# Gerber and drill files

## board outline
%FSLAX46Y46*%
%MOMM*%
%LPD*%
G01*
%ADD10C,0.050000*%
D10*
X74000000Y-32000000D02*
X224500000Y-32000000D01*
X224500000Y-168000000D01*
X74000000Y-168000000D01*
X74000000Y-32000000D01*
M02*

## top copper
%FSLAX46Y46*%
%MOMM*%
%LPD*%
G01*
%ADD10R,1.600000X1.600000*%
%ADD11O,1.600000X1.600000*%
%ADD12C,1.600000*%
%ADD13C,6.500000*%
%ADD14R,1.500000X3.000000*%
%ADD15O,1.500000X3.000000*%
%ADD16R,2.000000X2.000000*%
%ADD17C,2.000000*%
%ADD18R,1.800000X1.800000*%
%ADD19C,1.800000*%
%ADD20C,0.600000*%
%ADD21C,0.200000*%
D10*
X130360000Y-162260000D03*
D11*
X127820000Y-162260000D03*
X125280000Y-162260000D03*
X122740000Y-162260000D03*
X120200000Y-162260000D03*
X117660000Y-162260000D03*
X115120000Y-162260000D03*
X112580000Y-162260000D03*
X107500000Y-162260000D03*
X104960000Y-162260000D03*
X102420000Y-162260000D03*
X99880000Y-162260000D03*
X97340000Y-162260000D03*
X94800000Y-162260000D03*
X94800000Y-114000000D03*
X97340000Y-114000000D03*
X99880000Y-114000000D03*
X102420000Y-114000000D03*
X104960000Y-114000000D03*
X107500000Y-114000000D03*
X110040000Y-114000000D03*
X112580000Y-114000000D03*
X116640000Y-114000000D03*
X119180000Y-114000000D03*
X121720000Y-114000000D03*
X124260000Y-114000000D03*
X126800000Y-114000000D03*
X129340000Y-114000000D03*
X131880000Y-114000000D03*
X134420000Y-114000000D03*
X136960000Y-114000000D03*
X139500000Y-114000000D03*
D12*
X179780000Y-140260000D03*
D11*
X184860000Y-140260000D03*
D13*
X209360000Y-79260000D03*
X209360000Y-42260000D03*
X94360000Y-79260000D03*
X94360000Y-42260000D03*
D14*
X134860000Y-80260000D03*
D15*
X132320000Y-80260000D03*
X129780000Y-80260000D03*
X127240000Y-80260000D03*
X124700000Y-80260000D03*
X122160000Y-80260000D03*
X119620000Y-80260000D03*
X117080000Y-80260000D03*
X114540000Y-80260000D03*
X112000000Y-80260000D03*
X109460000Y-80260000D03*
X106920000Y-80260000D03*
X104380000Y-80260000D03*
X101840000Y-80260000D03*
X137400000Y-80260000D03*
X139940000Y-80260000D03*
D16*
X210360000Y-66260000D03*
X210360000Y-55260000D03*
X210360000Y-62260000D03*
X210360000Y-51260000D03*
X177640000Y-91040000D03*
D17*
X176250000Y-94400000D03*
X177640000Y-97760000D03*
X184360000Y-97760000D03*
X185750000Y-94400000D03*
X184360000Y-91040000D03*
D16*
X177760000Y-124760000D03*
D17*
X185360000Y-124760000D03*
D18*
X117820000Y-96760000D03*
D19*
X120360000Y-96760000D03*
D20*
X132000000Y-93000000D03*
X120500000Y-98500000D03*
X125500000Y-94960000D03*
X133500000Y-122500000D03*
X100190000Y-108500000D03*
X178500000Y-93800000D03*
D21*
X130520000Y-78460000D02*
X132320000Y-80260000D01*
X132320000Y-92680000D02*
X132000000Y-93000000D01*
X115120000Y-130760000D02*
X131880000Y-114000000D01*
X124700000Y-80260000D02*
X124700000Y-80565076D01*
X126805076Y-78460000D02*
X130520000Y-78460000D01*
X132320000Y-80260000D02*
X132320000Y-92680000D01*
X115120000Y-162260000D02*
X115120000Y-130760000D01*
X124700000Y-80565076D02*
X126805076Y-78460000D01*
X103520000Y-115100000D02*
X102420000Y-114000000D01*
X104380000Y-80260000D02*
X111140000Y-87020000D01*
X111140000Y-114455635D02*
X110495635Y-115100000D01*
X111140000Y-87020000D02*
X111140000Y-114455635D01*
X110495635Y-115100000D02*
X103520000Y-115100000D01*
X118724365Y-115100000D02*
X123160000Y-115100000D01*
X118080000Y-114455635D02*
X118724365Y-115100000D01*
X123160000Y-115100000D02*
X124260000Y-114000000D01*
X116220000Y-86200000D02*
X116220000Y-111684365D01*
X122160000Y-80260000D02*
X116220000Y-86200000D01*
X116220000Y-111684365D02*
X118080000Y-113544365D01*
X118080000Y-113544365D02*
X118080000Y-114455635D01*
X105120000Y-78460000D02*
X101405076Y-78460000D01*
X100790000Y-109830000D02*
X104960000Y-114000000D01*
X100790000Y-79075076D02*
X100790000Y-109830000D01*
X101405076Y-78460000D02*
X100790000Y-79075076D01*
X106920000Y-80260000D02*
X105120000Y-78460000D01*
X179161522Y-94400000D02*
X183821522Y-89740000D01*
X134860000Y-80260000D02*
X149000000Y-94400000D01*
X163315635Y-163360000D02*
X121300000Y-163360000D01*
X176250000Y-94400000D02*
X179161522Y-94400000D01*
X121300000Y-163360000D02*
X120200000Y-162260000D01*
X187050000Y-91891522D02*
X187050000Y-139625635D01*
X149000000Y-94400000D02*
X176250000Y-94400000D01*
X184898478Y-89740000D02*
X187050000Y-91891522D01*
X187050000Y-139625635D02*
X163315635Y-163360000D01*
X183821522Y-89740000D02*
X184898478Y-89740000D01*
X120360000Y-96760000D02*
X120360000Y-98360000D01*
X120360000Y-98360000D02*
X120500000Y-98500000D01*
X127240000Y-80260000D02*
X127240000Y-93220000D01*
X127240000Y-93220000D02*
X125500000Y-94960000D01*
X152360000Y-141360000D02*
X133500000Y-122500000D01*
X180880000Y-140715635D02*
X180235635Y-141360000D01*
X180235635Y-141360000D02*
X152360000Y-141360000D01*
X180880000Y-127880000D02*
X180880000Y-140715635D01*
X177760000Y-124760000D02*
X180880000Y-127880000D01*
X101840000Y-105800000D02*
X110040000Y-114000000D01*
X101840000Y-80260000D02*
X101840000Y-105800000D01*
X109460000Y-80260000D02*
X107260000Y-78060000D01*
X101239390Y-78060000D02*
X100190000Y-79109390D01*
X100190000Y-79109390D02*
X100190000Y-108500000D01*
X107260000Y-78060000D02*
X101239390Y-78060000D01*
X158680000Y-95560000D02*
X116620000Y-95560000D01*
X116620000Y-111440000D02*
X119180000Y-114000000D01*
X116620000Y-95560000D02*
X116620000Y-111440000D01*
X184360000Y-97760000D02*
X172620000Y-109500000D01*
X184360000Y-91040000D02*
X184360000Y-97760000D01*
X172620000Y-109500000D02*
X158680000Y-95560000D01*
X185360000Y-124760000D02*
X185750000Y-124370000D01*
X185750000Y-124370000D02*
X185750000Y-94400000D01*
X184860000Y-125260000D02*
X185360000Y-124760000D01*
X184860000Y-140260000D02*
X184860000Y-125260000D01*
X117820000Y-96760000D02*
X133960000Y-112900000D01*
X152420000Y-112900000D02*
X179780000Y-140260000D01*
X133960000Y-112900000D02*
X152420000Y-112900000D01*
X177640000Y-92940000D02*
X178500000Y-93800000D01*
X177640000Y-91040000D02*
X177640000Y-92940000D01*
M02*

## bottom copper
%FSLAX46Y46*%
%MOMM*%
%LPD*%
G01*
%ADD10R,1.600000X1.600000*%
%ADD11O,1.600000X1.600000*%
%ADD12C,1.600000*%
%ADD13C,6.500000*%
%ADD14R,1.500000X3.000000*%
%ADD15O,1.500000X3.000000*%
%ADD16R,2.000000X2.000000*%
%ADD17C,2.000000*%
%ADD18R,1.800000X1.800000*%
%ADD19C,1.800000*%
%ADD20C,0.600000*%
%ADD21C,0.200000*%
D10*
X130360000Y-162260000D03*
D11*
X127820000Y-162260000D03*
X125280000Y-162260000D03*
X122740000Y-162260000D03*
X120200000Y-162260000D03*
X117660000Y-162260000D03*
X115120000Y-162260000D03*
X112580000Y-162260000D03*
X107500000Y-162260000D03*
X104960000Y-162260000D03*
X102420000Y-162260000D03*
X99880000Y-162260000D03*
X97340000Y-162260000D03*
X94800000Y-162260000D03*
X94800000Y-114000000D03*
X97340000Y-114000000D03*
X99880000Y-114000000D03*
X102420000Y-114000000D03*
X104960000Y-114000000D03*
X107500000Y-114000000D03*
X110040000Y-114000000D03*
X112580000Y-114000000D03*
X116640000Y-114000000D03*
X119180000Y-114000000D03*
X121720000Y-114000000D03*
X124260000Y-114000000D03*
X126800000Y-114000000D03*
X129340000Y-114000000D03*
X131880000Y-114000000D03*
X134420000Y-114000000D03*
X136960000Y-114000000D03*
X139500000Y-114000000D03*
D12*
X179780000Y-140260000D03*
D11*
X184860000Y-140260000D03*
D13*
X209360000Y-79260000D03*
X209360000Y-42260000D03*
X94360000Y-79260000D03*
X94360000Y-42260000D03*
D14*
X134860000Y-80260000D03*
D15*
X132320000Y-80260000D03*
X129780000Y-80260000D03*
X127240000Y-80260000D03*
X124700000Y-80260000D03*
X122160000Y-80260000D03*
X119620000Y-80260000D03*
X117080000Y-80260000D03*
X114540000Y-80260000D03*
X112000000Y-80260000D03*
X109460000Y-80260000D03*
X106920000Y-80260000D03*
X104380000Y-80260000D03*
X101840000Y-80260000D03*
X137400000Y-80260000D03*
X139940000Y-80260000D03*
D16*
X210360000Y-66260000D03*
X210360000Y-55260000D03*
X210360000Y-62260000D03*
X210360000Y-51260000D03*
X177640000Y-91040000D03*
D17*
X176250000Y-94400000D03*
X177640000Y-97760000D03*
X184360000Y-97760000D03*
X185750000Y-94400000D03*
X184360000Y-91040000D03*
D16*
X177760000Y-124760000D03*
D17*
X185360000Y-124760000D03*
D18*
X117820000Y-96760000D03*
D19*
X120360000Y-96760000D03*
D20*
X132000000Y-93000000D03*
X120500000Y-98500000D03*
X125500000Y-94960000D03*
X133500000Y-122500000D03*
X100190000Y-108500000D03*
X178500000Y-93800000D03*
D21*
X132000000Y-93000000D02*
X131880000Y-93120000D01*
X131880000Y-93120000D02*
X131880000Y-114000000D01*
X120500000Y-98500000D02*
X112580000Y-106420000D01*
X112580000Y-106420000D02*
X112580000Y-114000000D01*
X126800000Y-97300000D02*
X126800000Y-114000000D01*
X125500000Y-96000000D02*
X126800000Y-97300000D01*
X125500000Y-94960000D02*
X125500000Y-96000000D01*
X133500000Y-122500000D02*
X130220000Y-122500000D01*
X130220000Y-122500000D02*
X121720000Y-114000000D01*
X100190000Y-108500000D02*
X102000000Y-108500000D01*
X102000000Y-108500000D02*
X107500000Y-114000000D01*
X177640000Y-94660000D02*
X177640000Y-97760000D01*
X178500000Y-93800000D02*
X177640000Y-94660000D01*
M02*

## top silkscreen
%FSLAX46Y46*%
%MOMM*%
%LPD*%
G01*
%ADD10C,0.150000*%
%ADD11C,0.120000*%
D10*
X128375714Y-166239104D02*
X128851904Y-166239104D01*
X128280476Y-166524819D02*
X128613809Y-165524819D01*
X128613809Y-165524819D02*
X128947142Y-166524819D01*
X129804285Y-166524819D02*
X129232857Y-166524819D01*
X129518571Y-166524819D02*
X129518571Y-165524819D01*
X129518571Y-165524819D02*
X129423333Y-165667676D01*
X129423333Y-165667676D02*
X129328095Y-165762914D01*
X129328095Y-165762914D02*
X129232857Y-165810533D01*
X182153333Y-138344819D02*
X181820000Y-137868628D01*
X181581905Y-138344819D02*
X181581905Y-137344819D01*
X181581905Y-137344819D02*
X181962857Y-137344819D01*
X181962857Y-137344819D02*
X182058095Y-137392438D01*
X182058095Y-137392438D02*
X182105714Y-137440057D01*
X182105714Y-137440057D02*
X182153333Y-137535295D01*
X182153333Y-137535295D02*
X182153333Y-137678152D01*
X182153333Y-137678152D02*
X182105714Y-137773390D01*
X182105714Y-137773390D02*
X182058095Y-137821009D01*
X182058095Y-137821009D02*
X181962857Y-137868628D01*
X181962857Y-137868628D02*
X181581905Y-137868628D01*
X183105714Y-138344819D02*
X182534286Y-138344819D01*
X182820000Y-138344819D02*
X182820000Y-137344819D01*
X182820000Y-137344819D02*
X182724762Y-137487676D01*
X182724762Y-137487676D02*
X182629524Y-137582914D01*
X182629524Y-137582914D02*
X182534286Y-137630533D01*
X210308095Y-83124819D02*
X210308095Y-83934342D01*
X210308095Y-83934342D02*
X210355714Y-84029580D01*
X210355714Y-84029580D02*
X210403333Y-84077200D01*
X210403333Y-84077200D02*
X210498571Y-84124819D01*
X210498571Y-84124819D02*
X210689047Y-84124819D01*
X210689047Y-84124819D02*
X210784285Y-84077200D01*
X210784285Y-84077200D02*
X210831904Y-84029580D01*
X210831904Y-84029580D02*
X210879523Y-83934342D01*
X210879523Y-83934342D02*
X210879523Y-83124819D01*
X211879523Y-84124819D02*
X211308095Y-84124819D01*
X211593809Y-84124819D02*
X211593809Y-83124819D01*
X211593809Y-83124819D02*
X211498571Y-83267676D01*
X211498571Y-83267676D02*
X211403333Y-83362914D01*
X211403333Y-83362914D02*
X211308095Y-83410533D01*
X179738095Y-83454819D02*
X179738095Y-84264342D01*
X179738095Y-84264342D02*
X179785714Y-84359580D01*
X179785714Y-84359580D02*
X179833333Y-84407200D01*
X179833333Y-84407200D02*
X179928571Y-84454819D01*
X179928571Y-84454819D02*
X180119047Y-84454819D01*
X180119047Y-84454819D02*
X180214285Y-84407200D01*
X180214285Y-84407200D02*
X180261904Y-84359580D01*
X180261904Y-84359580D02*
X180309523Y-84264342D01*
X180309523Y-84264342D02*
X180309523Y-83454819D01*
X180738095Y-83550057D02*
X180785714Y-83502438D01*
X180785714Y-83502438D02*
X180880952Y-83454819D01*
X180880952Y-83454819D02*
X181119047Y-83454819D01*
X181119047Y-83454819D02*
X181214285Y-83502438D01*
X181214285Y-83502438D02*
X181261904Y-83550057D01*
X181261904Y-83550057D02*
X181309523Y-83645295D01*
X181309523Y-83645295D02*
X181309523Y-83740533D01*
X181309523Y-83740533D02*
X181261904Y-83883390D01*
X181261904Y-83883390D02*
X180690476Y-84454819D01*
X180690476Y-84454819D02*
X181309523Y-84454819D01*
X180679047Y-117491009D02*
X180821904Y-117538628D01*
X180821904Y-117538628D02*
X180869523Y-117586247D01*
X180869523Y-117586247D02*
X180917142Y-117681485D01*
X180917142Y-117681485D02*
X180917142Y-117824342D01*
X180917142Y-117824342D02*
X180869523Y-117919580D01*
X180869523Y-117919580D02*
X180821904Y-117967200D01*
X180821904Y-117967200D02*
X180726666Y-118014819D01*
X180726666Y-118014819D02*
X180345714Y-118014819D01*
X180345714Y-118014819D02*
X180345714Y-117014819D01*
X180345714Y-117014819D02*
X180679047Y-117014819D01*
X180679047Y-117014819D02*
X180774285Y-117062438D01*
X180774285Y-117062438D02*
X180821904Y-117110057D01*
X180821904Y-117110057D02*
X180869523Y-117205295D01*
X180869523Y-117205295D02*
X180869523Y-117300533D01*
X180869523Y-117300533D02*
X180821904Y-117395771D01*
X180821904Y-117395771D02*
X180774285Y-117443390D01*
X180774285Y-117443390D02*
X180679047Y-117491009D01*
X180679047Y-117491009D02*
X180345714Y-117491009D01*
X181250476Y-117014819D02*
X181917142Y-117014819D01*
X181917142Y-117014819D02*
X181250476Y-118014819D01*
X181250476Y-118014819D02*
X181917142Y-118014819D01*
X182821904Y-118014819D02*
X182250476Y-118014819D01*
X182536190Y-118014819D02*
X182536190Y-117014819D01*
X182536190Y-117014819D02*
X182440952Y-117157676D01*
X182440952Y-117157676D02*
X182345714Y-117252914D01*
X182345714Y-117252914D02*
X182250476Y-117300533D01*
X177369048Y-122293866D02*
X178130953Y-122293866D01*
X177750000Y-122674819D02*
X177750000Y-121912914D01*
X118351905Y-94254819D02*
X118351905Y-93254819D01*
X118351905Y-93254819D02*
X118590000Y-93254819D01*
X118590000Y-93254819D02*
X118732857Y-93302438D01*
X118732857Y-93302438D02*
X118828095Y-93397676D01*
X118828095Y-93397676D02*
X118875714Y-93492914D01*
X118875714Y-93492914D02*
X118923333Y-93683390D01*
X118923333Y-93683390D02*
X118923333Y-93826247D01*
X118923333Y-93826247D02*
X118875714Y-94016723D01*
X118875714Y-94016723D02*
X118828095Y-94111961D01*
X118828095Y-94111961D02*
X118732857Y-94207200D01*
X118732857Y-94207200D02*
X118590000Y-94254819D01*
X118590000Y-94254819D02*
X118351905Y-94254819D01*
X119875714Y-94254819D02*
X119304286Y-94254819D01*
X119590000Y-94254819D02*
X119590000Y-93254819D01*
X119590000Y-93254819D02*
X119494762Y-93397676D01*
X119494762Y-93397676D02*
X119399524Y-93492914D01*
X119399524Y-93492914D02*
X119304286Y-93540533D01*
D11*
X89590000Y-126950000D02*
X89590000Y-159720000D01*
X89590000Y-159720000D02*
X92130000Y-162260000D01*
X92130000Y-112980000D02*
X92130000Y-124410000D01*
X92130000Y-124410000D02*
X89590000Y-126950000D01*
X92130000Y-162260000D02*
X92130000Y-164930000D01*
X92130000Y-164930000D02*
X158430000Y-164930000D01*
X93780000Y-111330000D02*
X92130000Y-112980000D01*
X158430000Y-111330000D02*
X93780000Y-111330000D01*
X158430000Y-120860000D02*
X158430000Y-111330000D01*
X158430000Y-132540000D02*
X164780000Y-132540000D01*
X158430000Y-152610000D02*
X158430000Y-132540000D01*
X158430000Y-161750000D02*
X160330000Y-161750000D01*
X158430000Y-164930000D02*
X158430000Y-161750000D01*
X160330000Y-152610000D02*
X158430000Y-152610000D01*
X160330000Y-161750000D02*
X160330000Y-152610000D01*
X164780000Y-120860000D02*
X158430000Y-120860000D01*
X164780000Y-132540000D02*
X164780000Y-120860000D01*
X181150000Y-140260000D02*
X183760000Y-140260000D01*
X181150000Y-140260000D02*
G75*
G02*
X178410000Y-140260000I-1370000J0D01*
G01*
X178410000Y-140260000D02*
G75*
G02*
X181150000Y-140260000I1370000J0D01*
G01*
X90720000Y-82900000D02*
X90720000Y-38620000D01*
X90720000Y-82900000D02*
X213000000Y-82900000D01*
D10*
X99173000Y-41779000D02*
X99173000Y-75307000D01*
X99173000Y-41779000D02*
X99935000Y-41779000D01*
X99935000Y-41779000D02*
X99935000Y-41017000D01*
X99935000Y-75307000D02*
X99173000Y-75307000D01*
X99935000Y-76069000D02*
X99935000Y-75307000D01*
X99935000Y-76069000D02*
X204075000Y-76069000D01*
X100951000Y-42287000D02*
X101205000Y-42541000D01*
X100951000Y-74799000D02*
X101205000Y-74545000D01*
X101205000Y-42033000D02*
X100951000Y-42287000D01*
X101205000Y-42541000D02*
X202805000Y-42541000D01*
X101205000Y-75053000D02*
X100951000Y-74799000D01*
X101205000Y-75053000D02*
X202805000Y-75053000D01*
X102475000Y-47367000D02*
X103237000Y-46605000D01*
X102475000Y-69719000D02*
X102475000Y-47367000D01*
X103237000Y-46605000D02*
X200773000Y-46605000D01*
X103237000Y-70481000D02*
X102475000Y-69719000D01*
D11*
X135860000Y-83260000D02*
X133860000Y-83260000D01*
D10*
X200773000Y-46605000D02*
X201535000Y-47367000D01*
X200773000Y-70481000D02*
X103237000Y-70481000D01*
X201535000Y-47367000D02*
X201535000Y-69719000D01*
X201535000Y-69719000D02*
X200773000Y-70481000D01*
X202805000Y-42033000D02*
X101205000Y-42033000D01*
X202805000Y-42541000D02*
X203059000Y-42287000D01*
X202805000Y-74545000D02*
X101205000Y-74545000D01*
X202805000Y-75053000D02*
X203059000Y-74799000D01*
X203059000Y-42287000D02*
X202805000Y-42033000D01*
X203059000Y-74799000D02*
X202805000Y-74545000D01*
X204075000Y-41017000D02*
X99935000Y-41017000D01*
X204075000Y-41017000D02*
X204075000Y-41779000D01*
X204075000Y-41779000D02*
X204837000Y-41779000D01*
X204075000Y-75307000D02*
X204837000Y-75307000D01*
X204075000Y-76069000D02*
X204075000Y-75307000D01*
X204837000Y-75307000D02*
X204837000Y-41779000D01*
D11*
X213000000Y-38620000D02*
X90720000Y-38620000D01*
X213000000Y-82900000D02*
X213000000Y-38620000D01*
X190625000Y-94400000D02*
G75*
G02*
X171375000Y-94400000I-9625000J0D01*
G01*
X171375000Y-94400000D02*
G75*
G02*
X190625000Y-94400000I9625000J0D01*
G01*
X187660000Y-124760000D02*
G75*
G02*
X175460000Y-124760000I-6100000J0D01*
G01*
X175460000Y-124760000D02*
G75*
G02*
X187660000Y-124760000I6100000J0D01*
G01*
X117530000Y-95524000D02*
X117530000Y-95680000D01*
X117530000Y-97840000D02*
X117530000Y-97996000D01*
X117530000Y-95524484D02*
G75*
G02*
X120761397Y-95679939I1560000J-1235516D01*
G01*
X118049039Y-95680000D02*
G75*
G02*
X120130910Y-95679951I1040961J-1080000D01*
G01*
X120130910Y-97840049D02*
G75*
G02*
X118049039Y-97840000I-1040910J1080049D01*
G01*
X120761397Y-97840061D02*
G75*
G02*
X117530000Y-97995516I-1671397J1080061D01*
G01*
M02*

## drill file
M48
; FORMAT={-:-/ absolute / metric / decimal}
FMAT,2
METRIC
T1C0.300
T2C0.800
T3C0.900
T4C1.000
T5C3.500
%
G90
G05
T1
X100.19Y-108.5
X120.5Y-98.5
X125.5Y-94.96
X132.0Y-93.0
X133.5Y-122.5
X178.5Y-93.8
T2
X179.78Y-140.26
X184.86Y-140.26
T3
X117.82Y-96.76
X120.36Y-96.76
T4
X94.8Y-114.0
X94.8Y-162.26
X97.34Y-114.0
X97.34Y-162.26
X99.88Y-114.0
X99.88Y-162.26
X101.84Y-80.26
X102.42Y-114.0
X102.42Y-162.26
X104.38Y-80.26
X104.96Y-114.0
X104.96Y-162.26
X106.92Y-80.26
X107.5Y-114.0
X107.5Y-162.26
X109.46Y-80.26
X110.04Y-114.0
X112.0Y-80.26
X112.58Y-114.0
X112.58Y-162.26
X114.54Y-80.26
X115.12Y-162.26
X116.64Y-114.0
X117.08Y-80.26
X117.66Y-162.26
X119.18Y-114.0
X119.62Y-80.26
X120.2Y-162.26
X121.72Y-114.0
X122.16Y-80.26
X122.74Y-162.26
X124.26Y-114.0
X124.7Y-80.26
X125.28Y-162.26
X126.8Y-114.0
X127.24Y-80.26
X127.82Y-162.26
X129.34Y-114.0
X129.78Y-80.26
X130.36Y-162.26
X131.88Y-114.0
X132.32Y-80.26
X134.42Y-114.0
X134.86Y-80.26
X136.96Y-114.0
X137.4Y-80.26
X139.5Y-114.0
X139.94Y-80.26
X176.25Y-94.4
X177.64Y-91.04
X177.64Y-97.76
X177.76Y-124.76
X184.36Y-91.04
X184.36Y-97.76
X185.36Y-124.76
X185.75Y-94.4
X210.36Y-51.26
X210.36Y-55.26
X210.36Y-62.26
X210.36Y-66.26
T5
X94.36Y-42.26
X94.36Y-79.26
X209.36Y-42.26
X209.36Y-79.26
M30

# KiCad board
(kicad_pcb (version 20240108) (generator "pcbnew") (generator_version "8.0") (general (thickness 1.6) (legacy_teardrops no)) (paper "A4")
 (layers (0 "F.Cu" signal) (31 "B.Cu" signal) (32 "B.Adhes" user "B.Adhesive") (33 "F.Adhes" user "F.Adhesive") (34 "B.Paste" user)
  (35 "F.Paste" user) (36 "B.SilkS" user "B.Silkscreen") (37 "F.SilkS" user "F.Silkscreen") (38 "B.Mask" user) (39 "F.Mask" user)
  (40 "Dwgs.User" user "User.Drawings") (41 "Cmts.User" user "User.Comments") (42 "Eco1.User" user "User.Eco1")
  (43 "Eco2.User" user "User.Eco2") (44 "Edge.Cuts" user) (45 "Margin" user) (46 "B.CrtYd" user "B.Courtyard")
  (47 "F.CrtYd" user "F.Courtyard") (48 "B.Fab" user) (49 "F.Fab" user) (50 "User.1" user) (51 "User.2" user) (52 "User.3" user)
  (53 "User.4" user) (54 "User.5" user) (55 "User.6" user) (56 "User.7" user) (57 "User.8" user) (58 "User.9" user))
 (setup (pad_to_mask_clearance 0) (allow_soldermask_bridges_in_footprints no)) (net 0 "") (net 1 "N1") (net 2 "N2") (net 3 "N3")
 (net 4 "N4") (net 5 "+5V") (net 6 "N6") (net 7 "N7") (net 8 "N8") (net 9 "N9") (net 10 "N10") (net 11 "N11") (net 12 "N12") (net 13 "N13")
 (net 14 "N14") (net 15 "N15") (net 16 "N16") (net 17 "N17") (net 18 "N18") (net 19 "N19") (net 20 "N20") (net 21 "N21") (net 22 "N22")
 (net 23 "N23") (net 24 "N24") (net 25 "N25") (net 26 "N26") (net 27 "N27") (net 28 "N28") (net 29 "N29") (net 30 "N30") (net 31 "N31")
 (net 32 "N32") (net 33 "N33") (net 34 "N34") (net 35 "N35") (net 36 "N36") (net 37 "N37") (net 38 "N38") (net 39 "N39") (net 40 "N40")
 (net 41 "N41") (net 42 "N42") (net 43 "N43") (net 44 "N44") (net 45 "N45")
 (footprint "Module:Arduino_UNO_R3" (layer "F.Cu") (at 130.36 162.26 180)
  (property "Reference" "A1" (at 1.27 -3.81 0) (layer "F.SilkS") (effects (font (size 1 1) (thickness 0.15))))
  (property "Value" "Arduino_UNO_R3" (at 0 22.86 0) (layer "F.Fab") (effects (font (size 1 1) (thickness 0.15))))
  (fp_line (start 40.77 35.31) (end 40.77 2.54) (stroke (width 0.12) (type solid)) (layer "F.SilkS"))
  (fp_line (start 40.77 2.54) (end 38.23 0) (stroke (width 0.12) (type solid)) (layer "F.SilkS"))
  (fp_line (start 38.23 49.28) (end 38.23 37.85) (stroke (width 0.12) (type solid)) (layer "F.SilkS"))
  (fp_line (start 38.23 37.85) (end 40.77 35.31) (stroke (width 0.12) (type solid)) (layer "F.SilkS"))
  (fp_line (start 38.23 0) (end 38.23 -2.67) (stroke (width 0.12) (type solid)) (layer "F.SilkS"))
  (fp_line (start 38.23 -2.67) (end -28.07 -2.67) (stroke (width 0.12) (type solid)) (layer "F.SilkS"))
  (fp_line (start 36.58 50.93) (end 38.23 49.28) (stroke (width 0.12) (type solid)) (layer "F.SilkS"))
  (fp_line (start -28.07 50.93) (end 36.58 50.93) (stroke (width 0.12) (type solid)) (layer "F.SilkS"))
  (fp_line (start -28.07 41.4) (end -28.07 50.93) (stroke (width 0.12) (type solid)) (layer "F.SilkS"))
  (fp_line (start -28.07 29.72) (end -34.42 29.72) (stroke (width 0.12) (type solid)) (layer "F.SilkS"))
  (fp_line (start -28.07 9.65) (end -28.07 29.72) (stroke (width 0.12) (type solid)) (layer "F.SilkS"))
  (fp_line (start -28.07 0.51) (end -29.97 0.51) (stroke (width 0.12) (type solid)) (layer "F.SilkS"))
  (fp_line (start -28.07 -2.67) (end -28.07 0.51) (stroke (width 0.12) (type solid)) (layer "F.SilkS"))
  (fp_line (start -29.97 9.65) (end -28.07 9.65) (stroke (width 0.12) (type solid)) (layer "F.SilkS"))
  (fp_line (start -29.97 0.51) (end -29.97 9.65) (stroke (width 0.12) (type solid)) (layer "F.SilkS"))
  (fp_line (start -34.42 41.4) (end -28.07 41.4) (stroke (width 0.12) (type solid)) (layer "F.SilkS"))
  (fp_line (start -34.42 29.72) (end -34.42 41.4) (stroke (width 0.12) (type solid)) (layer "F.SilkS"))
  (pad "1" thru_hole rect (at 0 0 270) (size 1.6 1.6) (drill 1) (layers "*.Cu" "*.Mask") (remove_unused_layers no) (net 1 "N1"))
  (pad "2" thru_hole oval (at 2.54 0 270) (size 1.6 1.6) (drill 1) (layers "*.Cu" "*.Mask") (remove_unused_layers no) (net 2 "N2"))
  (pad "3" thru_hole oval (at 5.08 0 270) (size 1.6 1.6) (drill 1) (layers "*.Cu" "*.Mask") (remove_unused_layers no) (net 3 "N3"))
  (pad "4" thru_hole oval (at 7.62 0 270) (size 1.6 1.6) (drill 1) (layers "*.Cu" "*.Mask") (remove_unused_layers no) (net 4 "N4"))
  (pad "5" thru_hole oval (at 10.16 0 270) (size 1.6 1.6) (drill 1) (layers "*.Cu" "*.Mask") (remove_unused_layers no) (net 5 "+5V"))
  (pad "6" thru_hole oval (at 12.7 0 270) (size 1.6 1.6) (drill 1) (layers "*.Cu" "*.Mask") (remove_unused_layers no) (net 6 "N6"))
  (pad "7" thru_hole oval (at 15.24 0 270) (size 1.6 1.6) (drill 1) (layers "*.Cu" "*.Mask") (remove_unused_layers no) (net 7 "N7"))
  (pad "8" thru_hole oval (at 17.78 0 270) (size 1.6 1.6) (drill 1) (layers "*.Cu" "*.Mask") (remove_unused_layers no) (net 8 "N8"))
  (pad "9" thru_hole oval (at 22.86 0 270) (size 1.6 1.6) (drill 1) (layers "*.Cu" "*.Mask") (remove_unused_layers no) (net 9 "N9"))
  (pad "10" thru_hole oval (at 25.4 0 270) (size 1.6 1.6) (drill 1) (layers "*.Cu" "*.Mask") (remove_unused_layers no) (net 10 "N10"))
  (pad "11" thru_hole oval (at 27.94 0 270) (size 1.6 1.6) (drill 1) (layers "*.Cu" "*.Mask") (remove_unused_layers no) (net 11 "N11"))
  (pad "12" thru_hole oval (at 30.48 0 270) (size 1.6 1.6) (drill 1) (layers "*.Cu" "*.Mask") (remove_unused_layers no) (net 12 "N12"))
  (pad "13" thru_hole oval (at 33.02 0 270) (size 1.6 1.6) (drill 1) (layers "*.Cu" "*.Mask") (remove_unused_layers no) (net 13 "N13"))
  (pad "14" thru_hole oval (at 35.56 0 270) (size 1.6 1.6) (drill 1) (layers "*.Cu" "*.Mask") (remove_unused_layers no) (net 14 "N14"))
  (pad "15" thru_hole oval (at 35.56 48.26 270) (size 1.6 1.6) (drill 1) (layers "*.Cu" "*.Mask") (remove_unused_layers no) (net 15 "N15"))
  (pad "16" thru_hole oval (at 33.02 48.26 270) (size 1.6 1.6) (drill 1) (layers "*.Cu" "*.Mask") (remove_unused_layers no) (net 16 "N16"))
  (pad "17" thru_hole oval (at 30.48 48.26 270) (size 1.6 1.6) (drill 1) (layers "*.Cu" "*.Mask") (remove_unused_layers no) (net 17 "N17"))
  (pad "18" thru_hole oval (at 27.94 48.26 270) (size 1.6 1.6) (drill 1) (layers "*.Cu" "*.Mask") (remove_unused_layers no) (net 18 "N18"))
  (pad "19" thru_hole oval (at 25.4 48.26 270) (size 1.6 1.6) (drill 1) (layers "*.Cu" "*.Mask") (remove_unused_layers no) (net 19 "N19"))
  (pad "20" thru_hole oval (at 22.86 48.26 270) (size 1.6 1.6) (drill 1) (layers "*.Cu" "*.Mask") (remove_unused_layers no) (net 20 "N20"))
  (pad "21" thru_hole oval (at 20.32 48.26 270) (size 1.6 1.6) (drill 1) (layers "*.Cu" "*.Mask") (remove_unused_layers no) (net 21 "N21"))
  (pad "22" thru_hole oval (at 17.78 48.26 270) (size 1.6 1.6) (drill 1) (layers "*.Cu" "*.Mask") (remove_unused_layers no) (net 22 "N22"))
  (pad "23" thru_hole oval (at 13.72 48.26 270) (size 1.6 1.6) (drill 1) (layers "*.Cu" "*.Mask") (remove_unused_layers no) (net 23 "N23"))
  (pad "24" thru_hole oval (at 11.18 48.26 270) (size 1.6 1.6) (drill 1) (layers "*.Cu" "*.Mask") (remove_unused_layers no) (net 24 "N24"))
  (pad "25" thru_hole oval (at 8.64 48.26 270) (size 1.6 1.6) (drill 1) (layers "*.Cu" "*.Mask") (remove_unused_layers no) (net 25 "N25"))
  (pad "26" thru_hole oval (at 6.1 48.26 270) (size 1.6 1.6) (drill 1) (layers "*.Cu" "*.Mask") (remove_unused_layers no) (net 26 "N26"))
  (pad "27" thru_hole oval (at 3.56 48.26 270) (size 1.6 1.6) (drill 1) (layers "*.Cu" "*.Mask") (remove_unused_layers no) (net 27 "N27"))
  (pad "28" thru_hole oval (at 1.02 48.26 270) (size 1.6 1.6) (drill 1) (layers "*.Cu" "*.Mask") (remove_unused_layers no) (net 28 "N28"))
  (pad "29" thru_hole oval (at -1.52 48.26 270) (size 1.6 1.6) (drill 1) (layers "*.Cu" "*.Mask") (remove_unused_layers no) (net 7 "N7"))
  (pad "30" thru_hole oval (at -4.06 48.26 270) (size 1.6 1.6) (drill 1) (layers "*.Cu" "*.Mask") (remove_unused_layers no) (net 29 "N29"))
  (pad "31" thru_hole oval (at -6.6 48.26 270) (size 1.6 1.6) (drill 1) (layers "*.Cu" "*.Mask") (remove_unused_layers no) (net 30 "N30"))
  (pad "32" thru_hole oval (at -9.14 48.26 270) (size 1.6 1.6) (drill 1) (layers "*.Cu" "*.Mask") (remove_unused_layers no) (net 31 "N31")))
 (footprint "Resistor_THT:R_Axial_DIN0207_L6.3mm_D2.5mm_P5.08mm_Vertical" (layer "F.Cu") (at 179.78 140.26)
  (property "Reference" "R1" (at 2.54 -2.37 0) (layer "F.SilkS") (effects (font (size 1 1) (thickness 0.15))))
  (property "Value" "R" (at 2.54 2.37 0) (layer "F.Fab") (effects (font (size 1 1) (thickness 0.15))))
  (fp_line (start 1.37 0) (end 3.98 0) (stroke (width 0.12) (type solid)) (layer "F.SilkS"))
  (fp_circle (center 0 0) (end 1.37 0) (stroke (width 0.12) (type solid)) (fill none) (layer "F.SilkS"))
  (pad "1" thru_hole circle (at 0 0) (size 1.6 1.6) (drill 0.8) (layers "*.Cu" "*.Mask") (remove_unused_layers no) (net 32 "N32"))
  (pad "2" thru_hole oval (at 5.08 0) (size 1.6 1.6) (drill 0.8) (layers "*.Cu" "*.Mask") (remove_unused_layers no) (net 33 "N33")))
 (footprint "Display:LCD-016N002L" (layer "F.Cu") (at 134.86 80.26 180)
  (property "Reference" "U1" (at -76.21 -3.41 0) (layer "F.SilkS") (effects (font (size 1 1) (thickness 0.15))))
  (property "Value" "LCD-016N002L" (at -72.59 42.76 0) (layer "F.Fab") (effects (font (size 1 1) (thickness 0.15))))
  (fp_line (start 44.14 -2.64) (end 44.14 41.64) (stroke (width 0.12) (type solid)) (layer "F.SilkS"))
  (fp_line (start 44.14 -2.64) (end -78.14 -2.64) (stroke (width 0.12) (type solid)) (layer "F.SilkS"))
  (fp_line (start 35.687 38.481) (end 35.687 4.953) (stroke (width 0.15) (type solid)) (layer "F.SilkS"))
  (fp_line (start 35.687 38.481) (end 34.925 38.481) (stroke (width 0.15) (type solid)) (layer "F.SilkS"))
  (fp_line (start 34.925 38.481) (end 34.925 39.243) (stroke (width 0.15) (type solid)) (layer "F.SilkS"))
  (fp_line (start 34.925 4.953) (end 35.687 4.953) (stroke (width 0.15) (type solid)) (layer "F.SilkS"))
  (fp_line (start 34.925 4.191) (end 34.925 4.953) (stroke (width 0.15) (type solid)) (layer "F.SilkS"))
  (fp_line (start 34.925 4.191) (end -69.215 4.191) (stroke (width 0.15) (type solid)) (layer "F.SilkS"))
  (fp_line (start 33.909 37.973) (end 33.655 37.719) (stroke (width 0.15) (type solid)) (layer "F.SilkS"))
  (fp_line (start 33.909 5.461) (end 33.655 5.715) (stroke (width 0.15) (type solid)) (layer "F.SilkS"))
  (fp_line (start 33.655 38.227) (end 33.909 37.973) (stroke (width 0.15) (type solid)) (layer "F.SilkS"))
  (fp_line (start 33.655 37.719) (end -67.945 37.719) (stroke (width 0.15) (type solid)) (layer "F.SilkS"))
  (fp_line (start 33.655 5.207) (end 33.909 5.461) (stroke (width 0.15) (type solid)) (layer "F.SilkS"))
  (fp_line (start 33.655 5.207) (end -67.945 5.207) (stroke (width 0.15) (type solid)) (layer "F.SilkS"))
  (fp_line (start 32.385 32.893) (end 31.623 33.655) (stroke (width 0.15) (type solid)) (layer "F.SilkS"))
  (fp_line (start 32.385 10.541) (end 32.385 32.893) (stroke (width 0.15) (type solid)) (layer "F.SilkS"))
  (fp_line (start 31.623 33.655) (end -65.913 33.655) (stroke (width 0.15) (type solid)) (layer "F.SilkS"))
  (fp_line (start 31.623 9.779) (end 32.385 10.541) (stroke (width 0.15) (type solid)) (layer "F.SilkS"))
  (fp_line (start -1 -3) (end 1 -3) (stroke (width 0.12) (type solid)) (layer "F.SilkS"))
  (fp_line (start -65.913 33.655) (end -66.675 32.893) (stroke (width 0.15) (type solid)) (layer "F.SilkS"))
  (fp_line (start -65.913 9.779) (end 31.623 9.779) (stroke (width 0.15) (type solid)) (layer "F.SilkS"))
  (fp_line (start -66.675 32.893) (end -66.675 10.541) (stroke (width 0.15) (type solid)) (layer "F.SilkS"))
  (fp_line (start -66.675 10.541) (end -65.913 9.779) (stroke (width 0.15) (type solid)) (layer "F.SilkS"))
  (fp_line (start -67.945 38.227) (end 33.655 38.227) (stroke (width 0.15) (type solid)) (layer "F.SilkS"))
  (fp_line (start -67.945 37.719) (end -68.199 37.973) (stroke (width 0.15) (type solid)) (layer "F.SilkS"))
  (fp_line (start -67.945 5.715) (end 33.655 5.715) (stroke (width 0.15) (type solid)) (layer "F.SilkS"))
  (fp_line (start -67.945 5.207) (end -68.199 5.461) (stroke (width 0.15) (type solid)) (layer "F.SilkS"))
  (fp_line (start -68.199 37.973) (end -67.945 38.227) (stroke (width 0.15) (type solid)) (layer "F.SilkS"))
  (fp_line (start -68.199 5.461) (end -67.945 5.715) (stroke (width 0.15) (type solid)) (layer "F.SilkS"))
  (fp_line (start -69.215 39.243) (end 34.925 39.243) (stroke (width 0.15) (type solid)) (layer "F.SilkS"))
  (fp_line (start -69.215 39.243) (end -69.215 38.481) (stroke (width 0.15) (type solid)) (layer "F.SilkS"))
  (fp_line (start -69.215 38.481) (end -69.977 38.481) (stroke (width 0.15) (type solid)) (layer "F.SilkS"))
  (fp_line (start -69.215 4.953) (end -69.977 4.953) (stroke (width 0.15) (type solid)) (layer "F.SilkS"))
  (fp_line (start -69.215 4.191) (end -69.215 4.953) (stroke (width 0.15) (type solid)) (layer "F.SilkS"))
  (fp_line (start -69.977 4.953) (end -69.977 38.481) (stroke (width 0.15) (type solid)) (layer "F.SilkS"))
  (fp_line (start -78.14 41.64) (end 44.14 41.64) (stroke (width 0.12) (type solid)) (layer "F.SilkS"))
  (fp_line (start -78.14 -2.64) (end -78.14 41.64) (stroke (width 0.12) (type solid)) (layer "F.SilkS"))
  (pad "" thru_hole circle (at -74.5 1) (size 6.5 6.5) (drill 3.5) (layers "*.Cu" "*.Mask") (remove_unused_layers no))
  (pad "" thru_hole circle (at -74.5 38) (size 6.5 6.5) (drill 3.5) (layers "*.Cu" "*.Mask") (remove_unused_layers no))
  (pad "" thru_hole circle (at 40.5 1) (size 6.5 6.5) (drill 3.5) (layers "*.Cu" "*.Mask") (remove_unused_layers no))
  (pad "" thru_hole circle (at 40.5 38) (size 6.5 6.5) (drill 3.5) (layers "*.Cu" "*.Mask") (remove_unused_layers no))
  (pad "1" thru_hole rect (at 0 0) (size 1.5 3) (drill 1) (layers "*.Cu" "*.Mask") (remove_unused_layers no) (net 5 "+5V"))
  (pad "2" thru_hole oval (at 2.54 0) (size 1.5 3) (drill 1) (layers "*.Cu" "*.Mask") (remove_unused_layers no) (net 7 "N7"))
  (pad "3" thru_hole oval (at 5.08 0) (size 1.5 3) (drill 1) (layers "*.Cu" "*.Mask") (remove_unused_layers no) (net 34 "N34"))
  (pad "4" thru_hole oval (at 7.62 0) (size 1.5 3) (drill 1) (layers "*.Cu" "*.Mask") (remove_unused_layers no) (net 27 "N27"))
  (pad "5" thru_hole oval (at 10.16 0) (size 1.5 3) (drill 1) (layers "*.Cu" "*.Mask") (remove_unused_layers no) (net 7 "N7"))
  (pad "6" thru_hole oval (at 12.7 0) (size 1.5 3) (drill 1) (layers "*.Cu" "*.Mask") (remove_unused_layers no) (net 26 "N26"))
  (pad "7" thru_hole oval (at 15.24 0) (size 1.5 3) (drill 1) (layers "*.Cu" "*.Mask") (remove_unused_layers no) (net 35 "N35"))
  (pad "8" thru_hole oval (at 17.78 0) (size 1.5 3) (drill 1) (layers "*.Cu" "*.Mask") (remove_unused_layers no) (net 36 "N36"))
  (pad "9" thru_hole oval (at 20.32 0) (size 1.5 3) (drill 1) (layers "*.Cu" "*.Mask") (remove_unused_layers no) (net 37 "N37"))
  (pad "10" thru_hole oval (at 22.86 0) (size 1.5 3) (drill 1) (layers "*.Cu" "*.Mask") (remove_unused_layers no) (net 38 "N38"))
  (pad "11" thru_hole oval (at 25.4 0) (size 1.5 3) (drill 1) (layers "*.Cu" "*.Mask") (remove_unused_layers no) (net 20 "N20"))
  (pad "12" thru_hole oval (at 27.94 0) (size 1.5 3) (drill 1) (layers "*.Cu" "*.Mask") (remove_unused_layers no) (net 19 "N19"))
  (pad "13" thru_hole oval (at 30.48 0) (size 1.5 3) (drill 1) (layers "*.Cu" "*.Mask") (remove_unused_layers no) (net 18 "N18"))
  (pad "14" thru_hole oval (at 33.02 0) (size 1.5 3) (drill 1) (layers "*.Cu" "*.Mask") (remove_unused_layers no) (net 21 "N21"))
  (pad "15" thru_hole oval (at -2.54 0) (size 1.5 3) (drill 1) (layers "*.Cu" "*.Mask") (remove_unused_layers no) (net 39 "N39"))
  (pad "16" thru_hole oval (at -5.08 0) (size 1.5 3) (drill 1) (layers "*.Cu" "*.Mask") (remove_unused_layers no) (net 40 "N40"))
  (pad "A1" thru_hole rect (at -75.5 14) (size 2 2) (drill 1) (layers "*.Cu" "*.Mask") (remove_unused_layers no) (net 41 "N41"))
  (pad "A2" thru_hole rect (at -75.5 25) (size 2 2) (drill 1) (layers "*.Cu" "*.Mask") (remove_unused_layers no) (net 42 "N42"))
  (pad "K1" thru_hole rect (at -75.5 18) (size 2 2) (drill 1) (layers "*.Cu" "*.Mask") (remove_unused_layers no) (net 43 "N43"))
  (pad "K2" thru_hole rect (at -75.5 29) (size 2 2) (drill 1) (layers "*.Cu" "*.Mask") (remove_unused_layers no) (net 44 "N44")))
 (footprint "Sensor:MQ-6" (layer "F.Cu") (at 177.64 91.04)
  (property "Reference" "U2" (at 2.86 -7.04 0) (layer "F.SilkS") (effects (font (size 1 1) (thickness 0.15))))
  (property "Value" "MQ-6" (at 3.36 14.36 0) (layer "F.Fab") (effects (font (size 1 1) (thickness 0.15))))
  (fp_circle (center 3.36 3.36) (end 12.985 3.36) (stroke (width 0.12) (type solid)) (fill none) (layer "F.SilkS"))
  (pad "1" thru_hole rect (at 0 0) (size 2 2) (drill 1) (layers "*.Cu" "*.Mask") (remove_unused_layers no) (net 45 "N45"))
  (pad "2" thru_hole circle (at -1.39 3.36) (size 2 2) (drill 1) (layers "*.Cu" "*.Mask") (remove_unused_layers no) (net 5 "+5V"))
  (pad "3" thru_hole circle (at 0 6.72 90) (size 2 2) (drill 1) (layers "*.Cu" "*.Mask") (remove_unused_layers no) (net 45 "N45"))
  (pad "4" thru_hole circle (at 6.72 6.72 180) (size 2 2) (drill 1) (layers "*.Cu" "*.Mask") (remove_unused_layers no) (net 24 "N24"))
  (pad "5" thru_hole circle (at 8.11 3.36) (size 2 2) (drill 1) (layers "*.Cu" "*.Mask") (remove_unused_layers no) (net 33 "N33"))
  (pad "6" thru_hole circle (at 6.72 0 270) (size 2 2) (drill 1) (layers "*.Cu" "*.Mask") (remove_unused_layers no) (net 24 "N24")))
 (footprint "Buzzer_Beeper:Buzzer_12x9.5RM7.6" (layer "F.Cu") (at 177.76 124.76)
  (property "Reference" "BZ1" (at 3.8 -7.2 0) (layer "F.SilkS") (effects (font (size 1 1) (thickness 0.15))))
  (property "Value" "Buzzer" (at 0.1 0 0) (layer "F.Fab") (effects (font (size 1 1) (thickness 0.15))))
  (fp_circle (center 3.8 0) (end 9.9 0) (stroke (width 0.12) (type solid)) (fill none) (layer "F.SilkS"))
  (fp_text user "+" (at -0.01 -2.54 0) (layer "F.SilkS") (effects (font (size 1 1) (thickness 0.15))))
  (pad "1" thru_hole rect (at 0 0) (size 2 2) (drill 1) (layers "*.Cu" "*.Mask") (remove_unused_layers no) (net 25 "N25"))
  (pad "2" thru_hole circle (at 7.6 0) (size 2 2) (drill 1) (layers "*.Cu" "*.Mask") (remove_unused_layers no) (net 33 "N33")))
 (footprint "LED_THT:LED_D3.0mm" (layer "F.Cu") (at 117.82 96.76)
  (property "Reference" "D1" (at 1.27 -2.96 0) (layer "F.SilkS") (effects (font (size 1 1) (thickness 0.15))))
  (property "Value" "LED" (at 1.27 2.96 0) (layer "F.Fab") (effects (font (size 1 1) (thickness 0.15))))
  (fp_line (start -0.29 -1.236) (end -0.29 -1.08) (stroke (width 0.12) (type solid)) (layer "F.SilkS"))
  (fp_line (start -0.29 1.08) (end -0.29 1.236) (stroke (width 0.12) (type solid)) (layer "F.SilkS"))
  (fp_arc (start -0.29 -1.235516) (mid 1.365624 -1.987701) (end 2.941397 -1.080061) (stroke (width 0.12) (type solid)) (layer "F.SilkS"))
  (fp_arc (start 0.229039 -1.08) (mid 1.269965 -1.5) (end 2.31091 -1.080049) (stroke (width 0.12) (type solid)) (layer "F.SilkS"))
  (fp_arc (start 2.31091 1.080049) (mid 1.269965 1.5) (end 0.229039 1.08) (stroke (width 0.12) (type solid)) (layer "F.SilkS"))
  (fp_arc (start 2.941397 1.080061) (mid 1.365624 1.987701) (end -0.29 1.235516) (stroke (width 0.12) (type solid)) (layer "F.SilkS"))
  (pad "1" thru_hole rect (at 0 0) (size 1.8 1.8) (drill 0.9) (layers "*.Cu" "*.Mask") (remove_unused_layers no) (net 32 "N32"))
  (pad "2" thru_hole circle (at 2.54 0) (size 1.8 1.8) (drill 0.9) (layers "*.Cu" "*.Mask") (remove_unused_layers no) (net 22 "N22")))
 (gr_rect (start 74 32) (end 224.5 168) (stroke (width 0.05) (type default)) (fill none) (layer "Edge.Cuts"))
 (segment (start 130.52 78.46) (end 132.32 80.26) (width 0.2) (layer "F.Cu") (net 7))
 (segment (start 132.32 92.68) (end 132 93) (width 0.2) (layer "F.Cu") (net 7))
 (segment (start 115.12 130.76) (end 131.88 114) (width 0.2) (layer "F.Cu") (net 7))
 (segment (start 124.7 80.26) (end 124.7 80.565076) (width 0.2) (layer "F.Cu") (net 7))
 (segment (start 126.805076 78.46) (end 130.52 78.46) (width 0.2) (layer "F.Cu") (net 7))
 (segment (start 132.32 80.26) (end 132.32 92.68) (width 0.2) (layer "F.Cu") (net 7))
 (segment (start 115.12 162.26) (end 115.12 130.76) (width 0.2) (layer "F.Cu") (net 7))
 (segment (start 124.7 80.565076) (end 126.805076 78.46) (width 0.2) (layer "F.Cu") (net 7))
 (via (at 132 93) (size 0.6) (drill 0.3) (layers "F.Cu" "B.Cu") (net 7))
 (segment (start 132 93) (end 131.88 93.12) (width 0.2) (layer "B.Cu") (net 7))
 (segment (start 131.88 93.12) (end 131.88 114) (width 0.2) (layer "B.Cu") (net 7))
 (segment (start 103.52 115.1) (end 102.42 114) (width 0.2) (layer "F.Cu") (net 18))
 (segment (start 104.38 80.26) (end 111.14 87.02) (width 0.2) (layer "F.Cu") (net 18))
 (segment (start 111.14 114.455635) (end 110.495635 115.1) (width 0.2) (layer "F.Cu") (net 18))
 (segment (start 111.14 87.02) (end 111.14 114.455635) (width 0.2) (layer "F.Cu") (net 18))
 (segment (start 110.495635 115.1) (end 103.52 115.1) (width 0.2) (layer "F.Cu") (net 18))
 (segment (start 118.724365 115.1) (end 123.16 115.1) (width 0.2) (layer "F.Cu") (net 26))
 (segment (start 118.08 114.455635) (end 118.724365 115.1) (width 0.2) (layer "F.Cu") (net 26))
 (segment (start 123.16 115.1) (end 124.26 114) (width 0.2) (layer "F.Cu") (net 26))
 (segment (start 116.22 86.2) (end 116.22 111.684365) (width 0.2) (layer "F.Cu") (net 26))
 (segment (start 122.16 80.26) (end 116.22 86.2) (width 0.2) (layer "F.Cu") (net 26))
 (segment (start 116.22 111.684365) (end 118.08 113.544365) (width 0.2) (layer "F.Cu") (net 26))
 (segment (start 118.08 113.544365) (end 118.08 114.455635) (width 0.2) (layer "F.Cu") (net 26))
 (segment (start 105.12 78.46) (end 101.405076 78.46) (width 0.2) (layer "F.Cu") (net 19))
 (segment (start 100.79 109.83) (end 104.96 114) (width 0.2) (layer "F.Cu") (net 19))
 (segment (start 100.79 79.075076) (end 100.79 109.83) (width 0.2) (layer "F.Cu") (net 19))
 (segment (start 101.405076 78.46) (end 100.79 79.075076) (width 0.2) (layer "F.Cu") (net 19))
 (segment (start 106.92 80.26) (end 105.12 78.46) (width 0.2) (layer "F.Cu") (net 19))
 (segment (start 179.161522 94.4) (end 183.821522 89.74) (width 0.2) (layer "F.Cu") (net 5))
 (segment (start 134.86 80.26) (end 149 94.4) (width 0.2) (layer "F.Cu") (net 5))
 (segment (start 163.315635 163.36) (end 121.3 163.36) (width 0.2) (layer "F.Cu") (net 5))
 (segment (start 176.25 94.4) (end 179.161522 94.4) (width 0.2) (layer "F.Cu") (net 5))
 (segment (start 121.3 163.36) (end 120.2 162.26) (width 0.2) (layer "F.Cu") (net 5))
 (segment (start 187.05 91.891522) (end 187.05 139.625635) (width 0.2) (layer "F.Cu") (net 5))
 (segment (start 149 94.4) (end 176.25 94.4) (width 0.2) (layer "F.Cu") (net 5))
 (segment (start 184.898478 89.74) (end 187.05 91.891522) (width 0.2) (layer "F.Cu") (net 5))
 (segment (start 187.05 139.625635) (end 163.315635 163.36) (width 0.2) (layer "F.Cu") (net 5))
 (segment (start 183.821522 89.74) (end 184.898478 89.74) (width 0.2) (layer "F.Cu") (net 5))
 (segment (start 120.36 96.76) (end 120.36 98.36) (width 0.2) (layer "F.Cu") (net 22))
 (segment (start 120.36 98.36) (end 120.5 98.5) (width 0.2) (layer "F.Cu") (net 22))
 (via (at 120.5 98.5) (size 0.6) (drill 0.3) (layers "F.Cu" "B.Cu") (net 22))
 (segment (start 120.5 98.5) (end 112.58 106.42) (width 0.2) (layer "B.Cu") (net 22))
 (segment (start 112.58 106.42) (end 112.58 114) (width 0.2) (layer "B.Cu") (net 22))
 (segment (start 127.24 80.26) (end 127.24 93.22) (width 0.2) (layer "F.Cu") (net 27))
 (segment (start 127.24 93.22) (end 125.5 94.96) (width 0.2) (layer "F.Cu") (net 27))
 (via (at 125.5 94.96) (size 0.6) (drill 0.3) (layers "F.Cu" "B.Cu") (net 27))
 (segment (start 126.8 97.3) (end 126.8 114) (width 0.2) (layer "B.Cu") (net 27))
 (segment (start 125.5 96) (end 126.8 97.3) (width 0.2) (layer "B.Cu") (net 27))
 (segment (start 125.5 94.96) (end 125.5 96) (width 0.2) (layer "B.Cu") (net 27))
 (segment (start 152.36 141.36) (end 133.5 122.5) (width 0.2) (layer "F.Cu") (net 25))
 (segment (start 180.88 140.715635) (end 180.235635 141.36) (width 0.2) (layer "F.Cu") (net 25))
 (segment (start 180.235635 141.36) (end 152.36 141.36) (width 0.2) (layer "F.Cu") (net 25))
 (segment (start 180.88 127.88) (end 180.88 140.715635) (width 0.2) (layer "F.Cu") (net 25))
 (segment (start 177.76 124.76) (end 180.88 127.88) (width 0.2) (layer "F.Cu") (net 25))
 (via (at 133.5 122.5) (size 0.6) (drill 0.3) (layers "F.Cu" "B.Cu") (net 25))
 (segment (start 133.5 122.5) (end 130.22 122.5) (width 0.2) (layer "B.Cu") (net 25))
 (segment (start 130.22 122.5) (end 121.72 114) (width 0.2) (layer "B.Cu") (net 25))
 (segment (start 101.84 105.8) (end 110.04 114) (width 0.2) (layer "F.Cu") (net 21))
 (segment (start 101.84 80.26) (end 101.84 105.8) (width 0.2) (layer "F.Cu") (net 21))
 (segment (start 109.46 80.26) (end 107.26 78.06) (width 0.2) (layer "F.Cu") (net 20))
 (segment (start 101.23939 78.06) (end 100.19 79.10939) (width 0.2) (layer "F.Cu") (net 20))
 (segment (start 100.19 79.10939) (end 100.19 108.5) (width 0.2) (layer "F.Cu") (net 20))
 (segment (start 107.26 78.06) (end 101.23939 78.06) (width 0.2) (layer "F.Cu") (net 20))
 (via (at 100.19 108.5) (size 0.6) (drill 0.3) (layers "F.Cu" "B.Cu") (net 20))
 (segment (start 100.19 108.5) (end 102 108.5) (width 0.2) (layer "B.Cu") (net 20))
 (segment (start 102 108.5) (end 107.5 114) (width 0.2) (layer "B.Cu") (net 20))
 (segment (start 158.68 95.56) (end 116.62 95.56) (width 0.2) (layer "F.Cu") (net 24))
 (segment (start 116.62 111.44) (end 119.18 114) (width 0.2) (layer "F.Cu") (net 24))
 (segment (start 116.62 95.56) (end 116.62 111.44) (width 0.2) (layer "F.Cu") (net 24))
 (segment (start 184.36 97.76) (end 172.62 109.5) (width 0.2) (layer "F.Cu") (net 24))
 (segment (start 184.36 91.04) (end 184.36 97.76) (width 0.2) (layer "F.Cu") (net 24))
 (segment (start 172.62 109.5) (end 158.68 95.56) (width 0.2) (layer "F.Cu") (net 24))
 (segment (start 185.36 124.76) (end 185.75 124.37) (width 0.2) (layer "F.Cu") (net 33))
 (segment (start 185.75 124.37) (end 185.75 94.4) (width 0.2) (layer "F.Cu") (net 33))
 (segment (start 184.86 125.26) (end 185.36 124.76) (width 0.2) (layer "F.Cu") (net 33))
 (segment (start 184.86 140.26) (end 184.86 125.26) (width 0.2) (layer "F.Cu") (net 33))
 (segment (start 117.82 96.76) (end 133.96 112.9) (width 0.2) (layer "F.Cu") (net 32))
 (segment (start 152.42 112.9) (end 179.78 140.26) (width 0.2) (layer "F.Cu") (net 32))
 (segment (start 133.96 112.9) (end 152.42 112.9) (width 0.2) (layer "F.Cu") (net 32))
 (segment (start 177.64 92.94) (end 178.5 93.8) (width 0.2) (layer "F.Cu") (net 45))
 (segment (start 177.64 91.04) (end 177.64 92.94) (width 0.2) (layer "F.Cu") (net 45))
 (via (at 178.5 93.8) (size 0.6) (drill 0.3) (layers "F.Cu" "B.Cu") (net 45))
 (segment (start 177.64 94.66) (end 177.64 97.76) (width 0.2) (layer "B.Cu") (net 45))
 (segment (start 178.5 93.8) (end 177.64 94.66) (width 0.2) (layer "B.Cu") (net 45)))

